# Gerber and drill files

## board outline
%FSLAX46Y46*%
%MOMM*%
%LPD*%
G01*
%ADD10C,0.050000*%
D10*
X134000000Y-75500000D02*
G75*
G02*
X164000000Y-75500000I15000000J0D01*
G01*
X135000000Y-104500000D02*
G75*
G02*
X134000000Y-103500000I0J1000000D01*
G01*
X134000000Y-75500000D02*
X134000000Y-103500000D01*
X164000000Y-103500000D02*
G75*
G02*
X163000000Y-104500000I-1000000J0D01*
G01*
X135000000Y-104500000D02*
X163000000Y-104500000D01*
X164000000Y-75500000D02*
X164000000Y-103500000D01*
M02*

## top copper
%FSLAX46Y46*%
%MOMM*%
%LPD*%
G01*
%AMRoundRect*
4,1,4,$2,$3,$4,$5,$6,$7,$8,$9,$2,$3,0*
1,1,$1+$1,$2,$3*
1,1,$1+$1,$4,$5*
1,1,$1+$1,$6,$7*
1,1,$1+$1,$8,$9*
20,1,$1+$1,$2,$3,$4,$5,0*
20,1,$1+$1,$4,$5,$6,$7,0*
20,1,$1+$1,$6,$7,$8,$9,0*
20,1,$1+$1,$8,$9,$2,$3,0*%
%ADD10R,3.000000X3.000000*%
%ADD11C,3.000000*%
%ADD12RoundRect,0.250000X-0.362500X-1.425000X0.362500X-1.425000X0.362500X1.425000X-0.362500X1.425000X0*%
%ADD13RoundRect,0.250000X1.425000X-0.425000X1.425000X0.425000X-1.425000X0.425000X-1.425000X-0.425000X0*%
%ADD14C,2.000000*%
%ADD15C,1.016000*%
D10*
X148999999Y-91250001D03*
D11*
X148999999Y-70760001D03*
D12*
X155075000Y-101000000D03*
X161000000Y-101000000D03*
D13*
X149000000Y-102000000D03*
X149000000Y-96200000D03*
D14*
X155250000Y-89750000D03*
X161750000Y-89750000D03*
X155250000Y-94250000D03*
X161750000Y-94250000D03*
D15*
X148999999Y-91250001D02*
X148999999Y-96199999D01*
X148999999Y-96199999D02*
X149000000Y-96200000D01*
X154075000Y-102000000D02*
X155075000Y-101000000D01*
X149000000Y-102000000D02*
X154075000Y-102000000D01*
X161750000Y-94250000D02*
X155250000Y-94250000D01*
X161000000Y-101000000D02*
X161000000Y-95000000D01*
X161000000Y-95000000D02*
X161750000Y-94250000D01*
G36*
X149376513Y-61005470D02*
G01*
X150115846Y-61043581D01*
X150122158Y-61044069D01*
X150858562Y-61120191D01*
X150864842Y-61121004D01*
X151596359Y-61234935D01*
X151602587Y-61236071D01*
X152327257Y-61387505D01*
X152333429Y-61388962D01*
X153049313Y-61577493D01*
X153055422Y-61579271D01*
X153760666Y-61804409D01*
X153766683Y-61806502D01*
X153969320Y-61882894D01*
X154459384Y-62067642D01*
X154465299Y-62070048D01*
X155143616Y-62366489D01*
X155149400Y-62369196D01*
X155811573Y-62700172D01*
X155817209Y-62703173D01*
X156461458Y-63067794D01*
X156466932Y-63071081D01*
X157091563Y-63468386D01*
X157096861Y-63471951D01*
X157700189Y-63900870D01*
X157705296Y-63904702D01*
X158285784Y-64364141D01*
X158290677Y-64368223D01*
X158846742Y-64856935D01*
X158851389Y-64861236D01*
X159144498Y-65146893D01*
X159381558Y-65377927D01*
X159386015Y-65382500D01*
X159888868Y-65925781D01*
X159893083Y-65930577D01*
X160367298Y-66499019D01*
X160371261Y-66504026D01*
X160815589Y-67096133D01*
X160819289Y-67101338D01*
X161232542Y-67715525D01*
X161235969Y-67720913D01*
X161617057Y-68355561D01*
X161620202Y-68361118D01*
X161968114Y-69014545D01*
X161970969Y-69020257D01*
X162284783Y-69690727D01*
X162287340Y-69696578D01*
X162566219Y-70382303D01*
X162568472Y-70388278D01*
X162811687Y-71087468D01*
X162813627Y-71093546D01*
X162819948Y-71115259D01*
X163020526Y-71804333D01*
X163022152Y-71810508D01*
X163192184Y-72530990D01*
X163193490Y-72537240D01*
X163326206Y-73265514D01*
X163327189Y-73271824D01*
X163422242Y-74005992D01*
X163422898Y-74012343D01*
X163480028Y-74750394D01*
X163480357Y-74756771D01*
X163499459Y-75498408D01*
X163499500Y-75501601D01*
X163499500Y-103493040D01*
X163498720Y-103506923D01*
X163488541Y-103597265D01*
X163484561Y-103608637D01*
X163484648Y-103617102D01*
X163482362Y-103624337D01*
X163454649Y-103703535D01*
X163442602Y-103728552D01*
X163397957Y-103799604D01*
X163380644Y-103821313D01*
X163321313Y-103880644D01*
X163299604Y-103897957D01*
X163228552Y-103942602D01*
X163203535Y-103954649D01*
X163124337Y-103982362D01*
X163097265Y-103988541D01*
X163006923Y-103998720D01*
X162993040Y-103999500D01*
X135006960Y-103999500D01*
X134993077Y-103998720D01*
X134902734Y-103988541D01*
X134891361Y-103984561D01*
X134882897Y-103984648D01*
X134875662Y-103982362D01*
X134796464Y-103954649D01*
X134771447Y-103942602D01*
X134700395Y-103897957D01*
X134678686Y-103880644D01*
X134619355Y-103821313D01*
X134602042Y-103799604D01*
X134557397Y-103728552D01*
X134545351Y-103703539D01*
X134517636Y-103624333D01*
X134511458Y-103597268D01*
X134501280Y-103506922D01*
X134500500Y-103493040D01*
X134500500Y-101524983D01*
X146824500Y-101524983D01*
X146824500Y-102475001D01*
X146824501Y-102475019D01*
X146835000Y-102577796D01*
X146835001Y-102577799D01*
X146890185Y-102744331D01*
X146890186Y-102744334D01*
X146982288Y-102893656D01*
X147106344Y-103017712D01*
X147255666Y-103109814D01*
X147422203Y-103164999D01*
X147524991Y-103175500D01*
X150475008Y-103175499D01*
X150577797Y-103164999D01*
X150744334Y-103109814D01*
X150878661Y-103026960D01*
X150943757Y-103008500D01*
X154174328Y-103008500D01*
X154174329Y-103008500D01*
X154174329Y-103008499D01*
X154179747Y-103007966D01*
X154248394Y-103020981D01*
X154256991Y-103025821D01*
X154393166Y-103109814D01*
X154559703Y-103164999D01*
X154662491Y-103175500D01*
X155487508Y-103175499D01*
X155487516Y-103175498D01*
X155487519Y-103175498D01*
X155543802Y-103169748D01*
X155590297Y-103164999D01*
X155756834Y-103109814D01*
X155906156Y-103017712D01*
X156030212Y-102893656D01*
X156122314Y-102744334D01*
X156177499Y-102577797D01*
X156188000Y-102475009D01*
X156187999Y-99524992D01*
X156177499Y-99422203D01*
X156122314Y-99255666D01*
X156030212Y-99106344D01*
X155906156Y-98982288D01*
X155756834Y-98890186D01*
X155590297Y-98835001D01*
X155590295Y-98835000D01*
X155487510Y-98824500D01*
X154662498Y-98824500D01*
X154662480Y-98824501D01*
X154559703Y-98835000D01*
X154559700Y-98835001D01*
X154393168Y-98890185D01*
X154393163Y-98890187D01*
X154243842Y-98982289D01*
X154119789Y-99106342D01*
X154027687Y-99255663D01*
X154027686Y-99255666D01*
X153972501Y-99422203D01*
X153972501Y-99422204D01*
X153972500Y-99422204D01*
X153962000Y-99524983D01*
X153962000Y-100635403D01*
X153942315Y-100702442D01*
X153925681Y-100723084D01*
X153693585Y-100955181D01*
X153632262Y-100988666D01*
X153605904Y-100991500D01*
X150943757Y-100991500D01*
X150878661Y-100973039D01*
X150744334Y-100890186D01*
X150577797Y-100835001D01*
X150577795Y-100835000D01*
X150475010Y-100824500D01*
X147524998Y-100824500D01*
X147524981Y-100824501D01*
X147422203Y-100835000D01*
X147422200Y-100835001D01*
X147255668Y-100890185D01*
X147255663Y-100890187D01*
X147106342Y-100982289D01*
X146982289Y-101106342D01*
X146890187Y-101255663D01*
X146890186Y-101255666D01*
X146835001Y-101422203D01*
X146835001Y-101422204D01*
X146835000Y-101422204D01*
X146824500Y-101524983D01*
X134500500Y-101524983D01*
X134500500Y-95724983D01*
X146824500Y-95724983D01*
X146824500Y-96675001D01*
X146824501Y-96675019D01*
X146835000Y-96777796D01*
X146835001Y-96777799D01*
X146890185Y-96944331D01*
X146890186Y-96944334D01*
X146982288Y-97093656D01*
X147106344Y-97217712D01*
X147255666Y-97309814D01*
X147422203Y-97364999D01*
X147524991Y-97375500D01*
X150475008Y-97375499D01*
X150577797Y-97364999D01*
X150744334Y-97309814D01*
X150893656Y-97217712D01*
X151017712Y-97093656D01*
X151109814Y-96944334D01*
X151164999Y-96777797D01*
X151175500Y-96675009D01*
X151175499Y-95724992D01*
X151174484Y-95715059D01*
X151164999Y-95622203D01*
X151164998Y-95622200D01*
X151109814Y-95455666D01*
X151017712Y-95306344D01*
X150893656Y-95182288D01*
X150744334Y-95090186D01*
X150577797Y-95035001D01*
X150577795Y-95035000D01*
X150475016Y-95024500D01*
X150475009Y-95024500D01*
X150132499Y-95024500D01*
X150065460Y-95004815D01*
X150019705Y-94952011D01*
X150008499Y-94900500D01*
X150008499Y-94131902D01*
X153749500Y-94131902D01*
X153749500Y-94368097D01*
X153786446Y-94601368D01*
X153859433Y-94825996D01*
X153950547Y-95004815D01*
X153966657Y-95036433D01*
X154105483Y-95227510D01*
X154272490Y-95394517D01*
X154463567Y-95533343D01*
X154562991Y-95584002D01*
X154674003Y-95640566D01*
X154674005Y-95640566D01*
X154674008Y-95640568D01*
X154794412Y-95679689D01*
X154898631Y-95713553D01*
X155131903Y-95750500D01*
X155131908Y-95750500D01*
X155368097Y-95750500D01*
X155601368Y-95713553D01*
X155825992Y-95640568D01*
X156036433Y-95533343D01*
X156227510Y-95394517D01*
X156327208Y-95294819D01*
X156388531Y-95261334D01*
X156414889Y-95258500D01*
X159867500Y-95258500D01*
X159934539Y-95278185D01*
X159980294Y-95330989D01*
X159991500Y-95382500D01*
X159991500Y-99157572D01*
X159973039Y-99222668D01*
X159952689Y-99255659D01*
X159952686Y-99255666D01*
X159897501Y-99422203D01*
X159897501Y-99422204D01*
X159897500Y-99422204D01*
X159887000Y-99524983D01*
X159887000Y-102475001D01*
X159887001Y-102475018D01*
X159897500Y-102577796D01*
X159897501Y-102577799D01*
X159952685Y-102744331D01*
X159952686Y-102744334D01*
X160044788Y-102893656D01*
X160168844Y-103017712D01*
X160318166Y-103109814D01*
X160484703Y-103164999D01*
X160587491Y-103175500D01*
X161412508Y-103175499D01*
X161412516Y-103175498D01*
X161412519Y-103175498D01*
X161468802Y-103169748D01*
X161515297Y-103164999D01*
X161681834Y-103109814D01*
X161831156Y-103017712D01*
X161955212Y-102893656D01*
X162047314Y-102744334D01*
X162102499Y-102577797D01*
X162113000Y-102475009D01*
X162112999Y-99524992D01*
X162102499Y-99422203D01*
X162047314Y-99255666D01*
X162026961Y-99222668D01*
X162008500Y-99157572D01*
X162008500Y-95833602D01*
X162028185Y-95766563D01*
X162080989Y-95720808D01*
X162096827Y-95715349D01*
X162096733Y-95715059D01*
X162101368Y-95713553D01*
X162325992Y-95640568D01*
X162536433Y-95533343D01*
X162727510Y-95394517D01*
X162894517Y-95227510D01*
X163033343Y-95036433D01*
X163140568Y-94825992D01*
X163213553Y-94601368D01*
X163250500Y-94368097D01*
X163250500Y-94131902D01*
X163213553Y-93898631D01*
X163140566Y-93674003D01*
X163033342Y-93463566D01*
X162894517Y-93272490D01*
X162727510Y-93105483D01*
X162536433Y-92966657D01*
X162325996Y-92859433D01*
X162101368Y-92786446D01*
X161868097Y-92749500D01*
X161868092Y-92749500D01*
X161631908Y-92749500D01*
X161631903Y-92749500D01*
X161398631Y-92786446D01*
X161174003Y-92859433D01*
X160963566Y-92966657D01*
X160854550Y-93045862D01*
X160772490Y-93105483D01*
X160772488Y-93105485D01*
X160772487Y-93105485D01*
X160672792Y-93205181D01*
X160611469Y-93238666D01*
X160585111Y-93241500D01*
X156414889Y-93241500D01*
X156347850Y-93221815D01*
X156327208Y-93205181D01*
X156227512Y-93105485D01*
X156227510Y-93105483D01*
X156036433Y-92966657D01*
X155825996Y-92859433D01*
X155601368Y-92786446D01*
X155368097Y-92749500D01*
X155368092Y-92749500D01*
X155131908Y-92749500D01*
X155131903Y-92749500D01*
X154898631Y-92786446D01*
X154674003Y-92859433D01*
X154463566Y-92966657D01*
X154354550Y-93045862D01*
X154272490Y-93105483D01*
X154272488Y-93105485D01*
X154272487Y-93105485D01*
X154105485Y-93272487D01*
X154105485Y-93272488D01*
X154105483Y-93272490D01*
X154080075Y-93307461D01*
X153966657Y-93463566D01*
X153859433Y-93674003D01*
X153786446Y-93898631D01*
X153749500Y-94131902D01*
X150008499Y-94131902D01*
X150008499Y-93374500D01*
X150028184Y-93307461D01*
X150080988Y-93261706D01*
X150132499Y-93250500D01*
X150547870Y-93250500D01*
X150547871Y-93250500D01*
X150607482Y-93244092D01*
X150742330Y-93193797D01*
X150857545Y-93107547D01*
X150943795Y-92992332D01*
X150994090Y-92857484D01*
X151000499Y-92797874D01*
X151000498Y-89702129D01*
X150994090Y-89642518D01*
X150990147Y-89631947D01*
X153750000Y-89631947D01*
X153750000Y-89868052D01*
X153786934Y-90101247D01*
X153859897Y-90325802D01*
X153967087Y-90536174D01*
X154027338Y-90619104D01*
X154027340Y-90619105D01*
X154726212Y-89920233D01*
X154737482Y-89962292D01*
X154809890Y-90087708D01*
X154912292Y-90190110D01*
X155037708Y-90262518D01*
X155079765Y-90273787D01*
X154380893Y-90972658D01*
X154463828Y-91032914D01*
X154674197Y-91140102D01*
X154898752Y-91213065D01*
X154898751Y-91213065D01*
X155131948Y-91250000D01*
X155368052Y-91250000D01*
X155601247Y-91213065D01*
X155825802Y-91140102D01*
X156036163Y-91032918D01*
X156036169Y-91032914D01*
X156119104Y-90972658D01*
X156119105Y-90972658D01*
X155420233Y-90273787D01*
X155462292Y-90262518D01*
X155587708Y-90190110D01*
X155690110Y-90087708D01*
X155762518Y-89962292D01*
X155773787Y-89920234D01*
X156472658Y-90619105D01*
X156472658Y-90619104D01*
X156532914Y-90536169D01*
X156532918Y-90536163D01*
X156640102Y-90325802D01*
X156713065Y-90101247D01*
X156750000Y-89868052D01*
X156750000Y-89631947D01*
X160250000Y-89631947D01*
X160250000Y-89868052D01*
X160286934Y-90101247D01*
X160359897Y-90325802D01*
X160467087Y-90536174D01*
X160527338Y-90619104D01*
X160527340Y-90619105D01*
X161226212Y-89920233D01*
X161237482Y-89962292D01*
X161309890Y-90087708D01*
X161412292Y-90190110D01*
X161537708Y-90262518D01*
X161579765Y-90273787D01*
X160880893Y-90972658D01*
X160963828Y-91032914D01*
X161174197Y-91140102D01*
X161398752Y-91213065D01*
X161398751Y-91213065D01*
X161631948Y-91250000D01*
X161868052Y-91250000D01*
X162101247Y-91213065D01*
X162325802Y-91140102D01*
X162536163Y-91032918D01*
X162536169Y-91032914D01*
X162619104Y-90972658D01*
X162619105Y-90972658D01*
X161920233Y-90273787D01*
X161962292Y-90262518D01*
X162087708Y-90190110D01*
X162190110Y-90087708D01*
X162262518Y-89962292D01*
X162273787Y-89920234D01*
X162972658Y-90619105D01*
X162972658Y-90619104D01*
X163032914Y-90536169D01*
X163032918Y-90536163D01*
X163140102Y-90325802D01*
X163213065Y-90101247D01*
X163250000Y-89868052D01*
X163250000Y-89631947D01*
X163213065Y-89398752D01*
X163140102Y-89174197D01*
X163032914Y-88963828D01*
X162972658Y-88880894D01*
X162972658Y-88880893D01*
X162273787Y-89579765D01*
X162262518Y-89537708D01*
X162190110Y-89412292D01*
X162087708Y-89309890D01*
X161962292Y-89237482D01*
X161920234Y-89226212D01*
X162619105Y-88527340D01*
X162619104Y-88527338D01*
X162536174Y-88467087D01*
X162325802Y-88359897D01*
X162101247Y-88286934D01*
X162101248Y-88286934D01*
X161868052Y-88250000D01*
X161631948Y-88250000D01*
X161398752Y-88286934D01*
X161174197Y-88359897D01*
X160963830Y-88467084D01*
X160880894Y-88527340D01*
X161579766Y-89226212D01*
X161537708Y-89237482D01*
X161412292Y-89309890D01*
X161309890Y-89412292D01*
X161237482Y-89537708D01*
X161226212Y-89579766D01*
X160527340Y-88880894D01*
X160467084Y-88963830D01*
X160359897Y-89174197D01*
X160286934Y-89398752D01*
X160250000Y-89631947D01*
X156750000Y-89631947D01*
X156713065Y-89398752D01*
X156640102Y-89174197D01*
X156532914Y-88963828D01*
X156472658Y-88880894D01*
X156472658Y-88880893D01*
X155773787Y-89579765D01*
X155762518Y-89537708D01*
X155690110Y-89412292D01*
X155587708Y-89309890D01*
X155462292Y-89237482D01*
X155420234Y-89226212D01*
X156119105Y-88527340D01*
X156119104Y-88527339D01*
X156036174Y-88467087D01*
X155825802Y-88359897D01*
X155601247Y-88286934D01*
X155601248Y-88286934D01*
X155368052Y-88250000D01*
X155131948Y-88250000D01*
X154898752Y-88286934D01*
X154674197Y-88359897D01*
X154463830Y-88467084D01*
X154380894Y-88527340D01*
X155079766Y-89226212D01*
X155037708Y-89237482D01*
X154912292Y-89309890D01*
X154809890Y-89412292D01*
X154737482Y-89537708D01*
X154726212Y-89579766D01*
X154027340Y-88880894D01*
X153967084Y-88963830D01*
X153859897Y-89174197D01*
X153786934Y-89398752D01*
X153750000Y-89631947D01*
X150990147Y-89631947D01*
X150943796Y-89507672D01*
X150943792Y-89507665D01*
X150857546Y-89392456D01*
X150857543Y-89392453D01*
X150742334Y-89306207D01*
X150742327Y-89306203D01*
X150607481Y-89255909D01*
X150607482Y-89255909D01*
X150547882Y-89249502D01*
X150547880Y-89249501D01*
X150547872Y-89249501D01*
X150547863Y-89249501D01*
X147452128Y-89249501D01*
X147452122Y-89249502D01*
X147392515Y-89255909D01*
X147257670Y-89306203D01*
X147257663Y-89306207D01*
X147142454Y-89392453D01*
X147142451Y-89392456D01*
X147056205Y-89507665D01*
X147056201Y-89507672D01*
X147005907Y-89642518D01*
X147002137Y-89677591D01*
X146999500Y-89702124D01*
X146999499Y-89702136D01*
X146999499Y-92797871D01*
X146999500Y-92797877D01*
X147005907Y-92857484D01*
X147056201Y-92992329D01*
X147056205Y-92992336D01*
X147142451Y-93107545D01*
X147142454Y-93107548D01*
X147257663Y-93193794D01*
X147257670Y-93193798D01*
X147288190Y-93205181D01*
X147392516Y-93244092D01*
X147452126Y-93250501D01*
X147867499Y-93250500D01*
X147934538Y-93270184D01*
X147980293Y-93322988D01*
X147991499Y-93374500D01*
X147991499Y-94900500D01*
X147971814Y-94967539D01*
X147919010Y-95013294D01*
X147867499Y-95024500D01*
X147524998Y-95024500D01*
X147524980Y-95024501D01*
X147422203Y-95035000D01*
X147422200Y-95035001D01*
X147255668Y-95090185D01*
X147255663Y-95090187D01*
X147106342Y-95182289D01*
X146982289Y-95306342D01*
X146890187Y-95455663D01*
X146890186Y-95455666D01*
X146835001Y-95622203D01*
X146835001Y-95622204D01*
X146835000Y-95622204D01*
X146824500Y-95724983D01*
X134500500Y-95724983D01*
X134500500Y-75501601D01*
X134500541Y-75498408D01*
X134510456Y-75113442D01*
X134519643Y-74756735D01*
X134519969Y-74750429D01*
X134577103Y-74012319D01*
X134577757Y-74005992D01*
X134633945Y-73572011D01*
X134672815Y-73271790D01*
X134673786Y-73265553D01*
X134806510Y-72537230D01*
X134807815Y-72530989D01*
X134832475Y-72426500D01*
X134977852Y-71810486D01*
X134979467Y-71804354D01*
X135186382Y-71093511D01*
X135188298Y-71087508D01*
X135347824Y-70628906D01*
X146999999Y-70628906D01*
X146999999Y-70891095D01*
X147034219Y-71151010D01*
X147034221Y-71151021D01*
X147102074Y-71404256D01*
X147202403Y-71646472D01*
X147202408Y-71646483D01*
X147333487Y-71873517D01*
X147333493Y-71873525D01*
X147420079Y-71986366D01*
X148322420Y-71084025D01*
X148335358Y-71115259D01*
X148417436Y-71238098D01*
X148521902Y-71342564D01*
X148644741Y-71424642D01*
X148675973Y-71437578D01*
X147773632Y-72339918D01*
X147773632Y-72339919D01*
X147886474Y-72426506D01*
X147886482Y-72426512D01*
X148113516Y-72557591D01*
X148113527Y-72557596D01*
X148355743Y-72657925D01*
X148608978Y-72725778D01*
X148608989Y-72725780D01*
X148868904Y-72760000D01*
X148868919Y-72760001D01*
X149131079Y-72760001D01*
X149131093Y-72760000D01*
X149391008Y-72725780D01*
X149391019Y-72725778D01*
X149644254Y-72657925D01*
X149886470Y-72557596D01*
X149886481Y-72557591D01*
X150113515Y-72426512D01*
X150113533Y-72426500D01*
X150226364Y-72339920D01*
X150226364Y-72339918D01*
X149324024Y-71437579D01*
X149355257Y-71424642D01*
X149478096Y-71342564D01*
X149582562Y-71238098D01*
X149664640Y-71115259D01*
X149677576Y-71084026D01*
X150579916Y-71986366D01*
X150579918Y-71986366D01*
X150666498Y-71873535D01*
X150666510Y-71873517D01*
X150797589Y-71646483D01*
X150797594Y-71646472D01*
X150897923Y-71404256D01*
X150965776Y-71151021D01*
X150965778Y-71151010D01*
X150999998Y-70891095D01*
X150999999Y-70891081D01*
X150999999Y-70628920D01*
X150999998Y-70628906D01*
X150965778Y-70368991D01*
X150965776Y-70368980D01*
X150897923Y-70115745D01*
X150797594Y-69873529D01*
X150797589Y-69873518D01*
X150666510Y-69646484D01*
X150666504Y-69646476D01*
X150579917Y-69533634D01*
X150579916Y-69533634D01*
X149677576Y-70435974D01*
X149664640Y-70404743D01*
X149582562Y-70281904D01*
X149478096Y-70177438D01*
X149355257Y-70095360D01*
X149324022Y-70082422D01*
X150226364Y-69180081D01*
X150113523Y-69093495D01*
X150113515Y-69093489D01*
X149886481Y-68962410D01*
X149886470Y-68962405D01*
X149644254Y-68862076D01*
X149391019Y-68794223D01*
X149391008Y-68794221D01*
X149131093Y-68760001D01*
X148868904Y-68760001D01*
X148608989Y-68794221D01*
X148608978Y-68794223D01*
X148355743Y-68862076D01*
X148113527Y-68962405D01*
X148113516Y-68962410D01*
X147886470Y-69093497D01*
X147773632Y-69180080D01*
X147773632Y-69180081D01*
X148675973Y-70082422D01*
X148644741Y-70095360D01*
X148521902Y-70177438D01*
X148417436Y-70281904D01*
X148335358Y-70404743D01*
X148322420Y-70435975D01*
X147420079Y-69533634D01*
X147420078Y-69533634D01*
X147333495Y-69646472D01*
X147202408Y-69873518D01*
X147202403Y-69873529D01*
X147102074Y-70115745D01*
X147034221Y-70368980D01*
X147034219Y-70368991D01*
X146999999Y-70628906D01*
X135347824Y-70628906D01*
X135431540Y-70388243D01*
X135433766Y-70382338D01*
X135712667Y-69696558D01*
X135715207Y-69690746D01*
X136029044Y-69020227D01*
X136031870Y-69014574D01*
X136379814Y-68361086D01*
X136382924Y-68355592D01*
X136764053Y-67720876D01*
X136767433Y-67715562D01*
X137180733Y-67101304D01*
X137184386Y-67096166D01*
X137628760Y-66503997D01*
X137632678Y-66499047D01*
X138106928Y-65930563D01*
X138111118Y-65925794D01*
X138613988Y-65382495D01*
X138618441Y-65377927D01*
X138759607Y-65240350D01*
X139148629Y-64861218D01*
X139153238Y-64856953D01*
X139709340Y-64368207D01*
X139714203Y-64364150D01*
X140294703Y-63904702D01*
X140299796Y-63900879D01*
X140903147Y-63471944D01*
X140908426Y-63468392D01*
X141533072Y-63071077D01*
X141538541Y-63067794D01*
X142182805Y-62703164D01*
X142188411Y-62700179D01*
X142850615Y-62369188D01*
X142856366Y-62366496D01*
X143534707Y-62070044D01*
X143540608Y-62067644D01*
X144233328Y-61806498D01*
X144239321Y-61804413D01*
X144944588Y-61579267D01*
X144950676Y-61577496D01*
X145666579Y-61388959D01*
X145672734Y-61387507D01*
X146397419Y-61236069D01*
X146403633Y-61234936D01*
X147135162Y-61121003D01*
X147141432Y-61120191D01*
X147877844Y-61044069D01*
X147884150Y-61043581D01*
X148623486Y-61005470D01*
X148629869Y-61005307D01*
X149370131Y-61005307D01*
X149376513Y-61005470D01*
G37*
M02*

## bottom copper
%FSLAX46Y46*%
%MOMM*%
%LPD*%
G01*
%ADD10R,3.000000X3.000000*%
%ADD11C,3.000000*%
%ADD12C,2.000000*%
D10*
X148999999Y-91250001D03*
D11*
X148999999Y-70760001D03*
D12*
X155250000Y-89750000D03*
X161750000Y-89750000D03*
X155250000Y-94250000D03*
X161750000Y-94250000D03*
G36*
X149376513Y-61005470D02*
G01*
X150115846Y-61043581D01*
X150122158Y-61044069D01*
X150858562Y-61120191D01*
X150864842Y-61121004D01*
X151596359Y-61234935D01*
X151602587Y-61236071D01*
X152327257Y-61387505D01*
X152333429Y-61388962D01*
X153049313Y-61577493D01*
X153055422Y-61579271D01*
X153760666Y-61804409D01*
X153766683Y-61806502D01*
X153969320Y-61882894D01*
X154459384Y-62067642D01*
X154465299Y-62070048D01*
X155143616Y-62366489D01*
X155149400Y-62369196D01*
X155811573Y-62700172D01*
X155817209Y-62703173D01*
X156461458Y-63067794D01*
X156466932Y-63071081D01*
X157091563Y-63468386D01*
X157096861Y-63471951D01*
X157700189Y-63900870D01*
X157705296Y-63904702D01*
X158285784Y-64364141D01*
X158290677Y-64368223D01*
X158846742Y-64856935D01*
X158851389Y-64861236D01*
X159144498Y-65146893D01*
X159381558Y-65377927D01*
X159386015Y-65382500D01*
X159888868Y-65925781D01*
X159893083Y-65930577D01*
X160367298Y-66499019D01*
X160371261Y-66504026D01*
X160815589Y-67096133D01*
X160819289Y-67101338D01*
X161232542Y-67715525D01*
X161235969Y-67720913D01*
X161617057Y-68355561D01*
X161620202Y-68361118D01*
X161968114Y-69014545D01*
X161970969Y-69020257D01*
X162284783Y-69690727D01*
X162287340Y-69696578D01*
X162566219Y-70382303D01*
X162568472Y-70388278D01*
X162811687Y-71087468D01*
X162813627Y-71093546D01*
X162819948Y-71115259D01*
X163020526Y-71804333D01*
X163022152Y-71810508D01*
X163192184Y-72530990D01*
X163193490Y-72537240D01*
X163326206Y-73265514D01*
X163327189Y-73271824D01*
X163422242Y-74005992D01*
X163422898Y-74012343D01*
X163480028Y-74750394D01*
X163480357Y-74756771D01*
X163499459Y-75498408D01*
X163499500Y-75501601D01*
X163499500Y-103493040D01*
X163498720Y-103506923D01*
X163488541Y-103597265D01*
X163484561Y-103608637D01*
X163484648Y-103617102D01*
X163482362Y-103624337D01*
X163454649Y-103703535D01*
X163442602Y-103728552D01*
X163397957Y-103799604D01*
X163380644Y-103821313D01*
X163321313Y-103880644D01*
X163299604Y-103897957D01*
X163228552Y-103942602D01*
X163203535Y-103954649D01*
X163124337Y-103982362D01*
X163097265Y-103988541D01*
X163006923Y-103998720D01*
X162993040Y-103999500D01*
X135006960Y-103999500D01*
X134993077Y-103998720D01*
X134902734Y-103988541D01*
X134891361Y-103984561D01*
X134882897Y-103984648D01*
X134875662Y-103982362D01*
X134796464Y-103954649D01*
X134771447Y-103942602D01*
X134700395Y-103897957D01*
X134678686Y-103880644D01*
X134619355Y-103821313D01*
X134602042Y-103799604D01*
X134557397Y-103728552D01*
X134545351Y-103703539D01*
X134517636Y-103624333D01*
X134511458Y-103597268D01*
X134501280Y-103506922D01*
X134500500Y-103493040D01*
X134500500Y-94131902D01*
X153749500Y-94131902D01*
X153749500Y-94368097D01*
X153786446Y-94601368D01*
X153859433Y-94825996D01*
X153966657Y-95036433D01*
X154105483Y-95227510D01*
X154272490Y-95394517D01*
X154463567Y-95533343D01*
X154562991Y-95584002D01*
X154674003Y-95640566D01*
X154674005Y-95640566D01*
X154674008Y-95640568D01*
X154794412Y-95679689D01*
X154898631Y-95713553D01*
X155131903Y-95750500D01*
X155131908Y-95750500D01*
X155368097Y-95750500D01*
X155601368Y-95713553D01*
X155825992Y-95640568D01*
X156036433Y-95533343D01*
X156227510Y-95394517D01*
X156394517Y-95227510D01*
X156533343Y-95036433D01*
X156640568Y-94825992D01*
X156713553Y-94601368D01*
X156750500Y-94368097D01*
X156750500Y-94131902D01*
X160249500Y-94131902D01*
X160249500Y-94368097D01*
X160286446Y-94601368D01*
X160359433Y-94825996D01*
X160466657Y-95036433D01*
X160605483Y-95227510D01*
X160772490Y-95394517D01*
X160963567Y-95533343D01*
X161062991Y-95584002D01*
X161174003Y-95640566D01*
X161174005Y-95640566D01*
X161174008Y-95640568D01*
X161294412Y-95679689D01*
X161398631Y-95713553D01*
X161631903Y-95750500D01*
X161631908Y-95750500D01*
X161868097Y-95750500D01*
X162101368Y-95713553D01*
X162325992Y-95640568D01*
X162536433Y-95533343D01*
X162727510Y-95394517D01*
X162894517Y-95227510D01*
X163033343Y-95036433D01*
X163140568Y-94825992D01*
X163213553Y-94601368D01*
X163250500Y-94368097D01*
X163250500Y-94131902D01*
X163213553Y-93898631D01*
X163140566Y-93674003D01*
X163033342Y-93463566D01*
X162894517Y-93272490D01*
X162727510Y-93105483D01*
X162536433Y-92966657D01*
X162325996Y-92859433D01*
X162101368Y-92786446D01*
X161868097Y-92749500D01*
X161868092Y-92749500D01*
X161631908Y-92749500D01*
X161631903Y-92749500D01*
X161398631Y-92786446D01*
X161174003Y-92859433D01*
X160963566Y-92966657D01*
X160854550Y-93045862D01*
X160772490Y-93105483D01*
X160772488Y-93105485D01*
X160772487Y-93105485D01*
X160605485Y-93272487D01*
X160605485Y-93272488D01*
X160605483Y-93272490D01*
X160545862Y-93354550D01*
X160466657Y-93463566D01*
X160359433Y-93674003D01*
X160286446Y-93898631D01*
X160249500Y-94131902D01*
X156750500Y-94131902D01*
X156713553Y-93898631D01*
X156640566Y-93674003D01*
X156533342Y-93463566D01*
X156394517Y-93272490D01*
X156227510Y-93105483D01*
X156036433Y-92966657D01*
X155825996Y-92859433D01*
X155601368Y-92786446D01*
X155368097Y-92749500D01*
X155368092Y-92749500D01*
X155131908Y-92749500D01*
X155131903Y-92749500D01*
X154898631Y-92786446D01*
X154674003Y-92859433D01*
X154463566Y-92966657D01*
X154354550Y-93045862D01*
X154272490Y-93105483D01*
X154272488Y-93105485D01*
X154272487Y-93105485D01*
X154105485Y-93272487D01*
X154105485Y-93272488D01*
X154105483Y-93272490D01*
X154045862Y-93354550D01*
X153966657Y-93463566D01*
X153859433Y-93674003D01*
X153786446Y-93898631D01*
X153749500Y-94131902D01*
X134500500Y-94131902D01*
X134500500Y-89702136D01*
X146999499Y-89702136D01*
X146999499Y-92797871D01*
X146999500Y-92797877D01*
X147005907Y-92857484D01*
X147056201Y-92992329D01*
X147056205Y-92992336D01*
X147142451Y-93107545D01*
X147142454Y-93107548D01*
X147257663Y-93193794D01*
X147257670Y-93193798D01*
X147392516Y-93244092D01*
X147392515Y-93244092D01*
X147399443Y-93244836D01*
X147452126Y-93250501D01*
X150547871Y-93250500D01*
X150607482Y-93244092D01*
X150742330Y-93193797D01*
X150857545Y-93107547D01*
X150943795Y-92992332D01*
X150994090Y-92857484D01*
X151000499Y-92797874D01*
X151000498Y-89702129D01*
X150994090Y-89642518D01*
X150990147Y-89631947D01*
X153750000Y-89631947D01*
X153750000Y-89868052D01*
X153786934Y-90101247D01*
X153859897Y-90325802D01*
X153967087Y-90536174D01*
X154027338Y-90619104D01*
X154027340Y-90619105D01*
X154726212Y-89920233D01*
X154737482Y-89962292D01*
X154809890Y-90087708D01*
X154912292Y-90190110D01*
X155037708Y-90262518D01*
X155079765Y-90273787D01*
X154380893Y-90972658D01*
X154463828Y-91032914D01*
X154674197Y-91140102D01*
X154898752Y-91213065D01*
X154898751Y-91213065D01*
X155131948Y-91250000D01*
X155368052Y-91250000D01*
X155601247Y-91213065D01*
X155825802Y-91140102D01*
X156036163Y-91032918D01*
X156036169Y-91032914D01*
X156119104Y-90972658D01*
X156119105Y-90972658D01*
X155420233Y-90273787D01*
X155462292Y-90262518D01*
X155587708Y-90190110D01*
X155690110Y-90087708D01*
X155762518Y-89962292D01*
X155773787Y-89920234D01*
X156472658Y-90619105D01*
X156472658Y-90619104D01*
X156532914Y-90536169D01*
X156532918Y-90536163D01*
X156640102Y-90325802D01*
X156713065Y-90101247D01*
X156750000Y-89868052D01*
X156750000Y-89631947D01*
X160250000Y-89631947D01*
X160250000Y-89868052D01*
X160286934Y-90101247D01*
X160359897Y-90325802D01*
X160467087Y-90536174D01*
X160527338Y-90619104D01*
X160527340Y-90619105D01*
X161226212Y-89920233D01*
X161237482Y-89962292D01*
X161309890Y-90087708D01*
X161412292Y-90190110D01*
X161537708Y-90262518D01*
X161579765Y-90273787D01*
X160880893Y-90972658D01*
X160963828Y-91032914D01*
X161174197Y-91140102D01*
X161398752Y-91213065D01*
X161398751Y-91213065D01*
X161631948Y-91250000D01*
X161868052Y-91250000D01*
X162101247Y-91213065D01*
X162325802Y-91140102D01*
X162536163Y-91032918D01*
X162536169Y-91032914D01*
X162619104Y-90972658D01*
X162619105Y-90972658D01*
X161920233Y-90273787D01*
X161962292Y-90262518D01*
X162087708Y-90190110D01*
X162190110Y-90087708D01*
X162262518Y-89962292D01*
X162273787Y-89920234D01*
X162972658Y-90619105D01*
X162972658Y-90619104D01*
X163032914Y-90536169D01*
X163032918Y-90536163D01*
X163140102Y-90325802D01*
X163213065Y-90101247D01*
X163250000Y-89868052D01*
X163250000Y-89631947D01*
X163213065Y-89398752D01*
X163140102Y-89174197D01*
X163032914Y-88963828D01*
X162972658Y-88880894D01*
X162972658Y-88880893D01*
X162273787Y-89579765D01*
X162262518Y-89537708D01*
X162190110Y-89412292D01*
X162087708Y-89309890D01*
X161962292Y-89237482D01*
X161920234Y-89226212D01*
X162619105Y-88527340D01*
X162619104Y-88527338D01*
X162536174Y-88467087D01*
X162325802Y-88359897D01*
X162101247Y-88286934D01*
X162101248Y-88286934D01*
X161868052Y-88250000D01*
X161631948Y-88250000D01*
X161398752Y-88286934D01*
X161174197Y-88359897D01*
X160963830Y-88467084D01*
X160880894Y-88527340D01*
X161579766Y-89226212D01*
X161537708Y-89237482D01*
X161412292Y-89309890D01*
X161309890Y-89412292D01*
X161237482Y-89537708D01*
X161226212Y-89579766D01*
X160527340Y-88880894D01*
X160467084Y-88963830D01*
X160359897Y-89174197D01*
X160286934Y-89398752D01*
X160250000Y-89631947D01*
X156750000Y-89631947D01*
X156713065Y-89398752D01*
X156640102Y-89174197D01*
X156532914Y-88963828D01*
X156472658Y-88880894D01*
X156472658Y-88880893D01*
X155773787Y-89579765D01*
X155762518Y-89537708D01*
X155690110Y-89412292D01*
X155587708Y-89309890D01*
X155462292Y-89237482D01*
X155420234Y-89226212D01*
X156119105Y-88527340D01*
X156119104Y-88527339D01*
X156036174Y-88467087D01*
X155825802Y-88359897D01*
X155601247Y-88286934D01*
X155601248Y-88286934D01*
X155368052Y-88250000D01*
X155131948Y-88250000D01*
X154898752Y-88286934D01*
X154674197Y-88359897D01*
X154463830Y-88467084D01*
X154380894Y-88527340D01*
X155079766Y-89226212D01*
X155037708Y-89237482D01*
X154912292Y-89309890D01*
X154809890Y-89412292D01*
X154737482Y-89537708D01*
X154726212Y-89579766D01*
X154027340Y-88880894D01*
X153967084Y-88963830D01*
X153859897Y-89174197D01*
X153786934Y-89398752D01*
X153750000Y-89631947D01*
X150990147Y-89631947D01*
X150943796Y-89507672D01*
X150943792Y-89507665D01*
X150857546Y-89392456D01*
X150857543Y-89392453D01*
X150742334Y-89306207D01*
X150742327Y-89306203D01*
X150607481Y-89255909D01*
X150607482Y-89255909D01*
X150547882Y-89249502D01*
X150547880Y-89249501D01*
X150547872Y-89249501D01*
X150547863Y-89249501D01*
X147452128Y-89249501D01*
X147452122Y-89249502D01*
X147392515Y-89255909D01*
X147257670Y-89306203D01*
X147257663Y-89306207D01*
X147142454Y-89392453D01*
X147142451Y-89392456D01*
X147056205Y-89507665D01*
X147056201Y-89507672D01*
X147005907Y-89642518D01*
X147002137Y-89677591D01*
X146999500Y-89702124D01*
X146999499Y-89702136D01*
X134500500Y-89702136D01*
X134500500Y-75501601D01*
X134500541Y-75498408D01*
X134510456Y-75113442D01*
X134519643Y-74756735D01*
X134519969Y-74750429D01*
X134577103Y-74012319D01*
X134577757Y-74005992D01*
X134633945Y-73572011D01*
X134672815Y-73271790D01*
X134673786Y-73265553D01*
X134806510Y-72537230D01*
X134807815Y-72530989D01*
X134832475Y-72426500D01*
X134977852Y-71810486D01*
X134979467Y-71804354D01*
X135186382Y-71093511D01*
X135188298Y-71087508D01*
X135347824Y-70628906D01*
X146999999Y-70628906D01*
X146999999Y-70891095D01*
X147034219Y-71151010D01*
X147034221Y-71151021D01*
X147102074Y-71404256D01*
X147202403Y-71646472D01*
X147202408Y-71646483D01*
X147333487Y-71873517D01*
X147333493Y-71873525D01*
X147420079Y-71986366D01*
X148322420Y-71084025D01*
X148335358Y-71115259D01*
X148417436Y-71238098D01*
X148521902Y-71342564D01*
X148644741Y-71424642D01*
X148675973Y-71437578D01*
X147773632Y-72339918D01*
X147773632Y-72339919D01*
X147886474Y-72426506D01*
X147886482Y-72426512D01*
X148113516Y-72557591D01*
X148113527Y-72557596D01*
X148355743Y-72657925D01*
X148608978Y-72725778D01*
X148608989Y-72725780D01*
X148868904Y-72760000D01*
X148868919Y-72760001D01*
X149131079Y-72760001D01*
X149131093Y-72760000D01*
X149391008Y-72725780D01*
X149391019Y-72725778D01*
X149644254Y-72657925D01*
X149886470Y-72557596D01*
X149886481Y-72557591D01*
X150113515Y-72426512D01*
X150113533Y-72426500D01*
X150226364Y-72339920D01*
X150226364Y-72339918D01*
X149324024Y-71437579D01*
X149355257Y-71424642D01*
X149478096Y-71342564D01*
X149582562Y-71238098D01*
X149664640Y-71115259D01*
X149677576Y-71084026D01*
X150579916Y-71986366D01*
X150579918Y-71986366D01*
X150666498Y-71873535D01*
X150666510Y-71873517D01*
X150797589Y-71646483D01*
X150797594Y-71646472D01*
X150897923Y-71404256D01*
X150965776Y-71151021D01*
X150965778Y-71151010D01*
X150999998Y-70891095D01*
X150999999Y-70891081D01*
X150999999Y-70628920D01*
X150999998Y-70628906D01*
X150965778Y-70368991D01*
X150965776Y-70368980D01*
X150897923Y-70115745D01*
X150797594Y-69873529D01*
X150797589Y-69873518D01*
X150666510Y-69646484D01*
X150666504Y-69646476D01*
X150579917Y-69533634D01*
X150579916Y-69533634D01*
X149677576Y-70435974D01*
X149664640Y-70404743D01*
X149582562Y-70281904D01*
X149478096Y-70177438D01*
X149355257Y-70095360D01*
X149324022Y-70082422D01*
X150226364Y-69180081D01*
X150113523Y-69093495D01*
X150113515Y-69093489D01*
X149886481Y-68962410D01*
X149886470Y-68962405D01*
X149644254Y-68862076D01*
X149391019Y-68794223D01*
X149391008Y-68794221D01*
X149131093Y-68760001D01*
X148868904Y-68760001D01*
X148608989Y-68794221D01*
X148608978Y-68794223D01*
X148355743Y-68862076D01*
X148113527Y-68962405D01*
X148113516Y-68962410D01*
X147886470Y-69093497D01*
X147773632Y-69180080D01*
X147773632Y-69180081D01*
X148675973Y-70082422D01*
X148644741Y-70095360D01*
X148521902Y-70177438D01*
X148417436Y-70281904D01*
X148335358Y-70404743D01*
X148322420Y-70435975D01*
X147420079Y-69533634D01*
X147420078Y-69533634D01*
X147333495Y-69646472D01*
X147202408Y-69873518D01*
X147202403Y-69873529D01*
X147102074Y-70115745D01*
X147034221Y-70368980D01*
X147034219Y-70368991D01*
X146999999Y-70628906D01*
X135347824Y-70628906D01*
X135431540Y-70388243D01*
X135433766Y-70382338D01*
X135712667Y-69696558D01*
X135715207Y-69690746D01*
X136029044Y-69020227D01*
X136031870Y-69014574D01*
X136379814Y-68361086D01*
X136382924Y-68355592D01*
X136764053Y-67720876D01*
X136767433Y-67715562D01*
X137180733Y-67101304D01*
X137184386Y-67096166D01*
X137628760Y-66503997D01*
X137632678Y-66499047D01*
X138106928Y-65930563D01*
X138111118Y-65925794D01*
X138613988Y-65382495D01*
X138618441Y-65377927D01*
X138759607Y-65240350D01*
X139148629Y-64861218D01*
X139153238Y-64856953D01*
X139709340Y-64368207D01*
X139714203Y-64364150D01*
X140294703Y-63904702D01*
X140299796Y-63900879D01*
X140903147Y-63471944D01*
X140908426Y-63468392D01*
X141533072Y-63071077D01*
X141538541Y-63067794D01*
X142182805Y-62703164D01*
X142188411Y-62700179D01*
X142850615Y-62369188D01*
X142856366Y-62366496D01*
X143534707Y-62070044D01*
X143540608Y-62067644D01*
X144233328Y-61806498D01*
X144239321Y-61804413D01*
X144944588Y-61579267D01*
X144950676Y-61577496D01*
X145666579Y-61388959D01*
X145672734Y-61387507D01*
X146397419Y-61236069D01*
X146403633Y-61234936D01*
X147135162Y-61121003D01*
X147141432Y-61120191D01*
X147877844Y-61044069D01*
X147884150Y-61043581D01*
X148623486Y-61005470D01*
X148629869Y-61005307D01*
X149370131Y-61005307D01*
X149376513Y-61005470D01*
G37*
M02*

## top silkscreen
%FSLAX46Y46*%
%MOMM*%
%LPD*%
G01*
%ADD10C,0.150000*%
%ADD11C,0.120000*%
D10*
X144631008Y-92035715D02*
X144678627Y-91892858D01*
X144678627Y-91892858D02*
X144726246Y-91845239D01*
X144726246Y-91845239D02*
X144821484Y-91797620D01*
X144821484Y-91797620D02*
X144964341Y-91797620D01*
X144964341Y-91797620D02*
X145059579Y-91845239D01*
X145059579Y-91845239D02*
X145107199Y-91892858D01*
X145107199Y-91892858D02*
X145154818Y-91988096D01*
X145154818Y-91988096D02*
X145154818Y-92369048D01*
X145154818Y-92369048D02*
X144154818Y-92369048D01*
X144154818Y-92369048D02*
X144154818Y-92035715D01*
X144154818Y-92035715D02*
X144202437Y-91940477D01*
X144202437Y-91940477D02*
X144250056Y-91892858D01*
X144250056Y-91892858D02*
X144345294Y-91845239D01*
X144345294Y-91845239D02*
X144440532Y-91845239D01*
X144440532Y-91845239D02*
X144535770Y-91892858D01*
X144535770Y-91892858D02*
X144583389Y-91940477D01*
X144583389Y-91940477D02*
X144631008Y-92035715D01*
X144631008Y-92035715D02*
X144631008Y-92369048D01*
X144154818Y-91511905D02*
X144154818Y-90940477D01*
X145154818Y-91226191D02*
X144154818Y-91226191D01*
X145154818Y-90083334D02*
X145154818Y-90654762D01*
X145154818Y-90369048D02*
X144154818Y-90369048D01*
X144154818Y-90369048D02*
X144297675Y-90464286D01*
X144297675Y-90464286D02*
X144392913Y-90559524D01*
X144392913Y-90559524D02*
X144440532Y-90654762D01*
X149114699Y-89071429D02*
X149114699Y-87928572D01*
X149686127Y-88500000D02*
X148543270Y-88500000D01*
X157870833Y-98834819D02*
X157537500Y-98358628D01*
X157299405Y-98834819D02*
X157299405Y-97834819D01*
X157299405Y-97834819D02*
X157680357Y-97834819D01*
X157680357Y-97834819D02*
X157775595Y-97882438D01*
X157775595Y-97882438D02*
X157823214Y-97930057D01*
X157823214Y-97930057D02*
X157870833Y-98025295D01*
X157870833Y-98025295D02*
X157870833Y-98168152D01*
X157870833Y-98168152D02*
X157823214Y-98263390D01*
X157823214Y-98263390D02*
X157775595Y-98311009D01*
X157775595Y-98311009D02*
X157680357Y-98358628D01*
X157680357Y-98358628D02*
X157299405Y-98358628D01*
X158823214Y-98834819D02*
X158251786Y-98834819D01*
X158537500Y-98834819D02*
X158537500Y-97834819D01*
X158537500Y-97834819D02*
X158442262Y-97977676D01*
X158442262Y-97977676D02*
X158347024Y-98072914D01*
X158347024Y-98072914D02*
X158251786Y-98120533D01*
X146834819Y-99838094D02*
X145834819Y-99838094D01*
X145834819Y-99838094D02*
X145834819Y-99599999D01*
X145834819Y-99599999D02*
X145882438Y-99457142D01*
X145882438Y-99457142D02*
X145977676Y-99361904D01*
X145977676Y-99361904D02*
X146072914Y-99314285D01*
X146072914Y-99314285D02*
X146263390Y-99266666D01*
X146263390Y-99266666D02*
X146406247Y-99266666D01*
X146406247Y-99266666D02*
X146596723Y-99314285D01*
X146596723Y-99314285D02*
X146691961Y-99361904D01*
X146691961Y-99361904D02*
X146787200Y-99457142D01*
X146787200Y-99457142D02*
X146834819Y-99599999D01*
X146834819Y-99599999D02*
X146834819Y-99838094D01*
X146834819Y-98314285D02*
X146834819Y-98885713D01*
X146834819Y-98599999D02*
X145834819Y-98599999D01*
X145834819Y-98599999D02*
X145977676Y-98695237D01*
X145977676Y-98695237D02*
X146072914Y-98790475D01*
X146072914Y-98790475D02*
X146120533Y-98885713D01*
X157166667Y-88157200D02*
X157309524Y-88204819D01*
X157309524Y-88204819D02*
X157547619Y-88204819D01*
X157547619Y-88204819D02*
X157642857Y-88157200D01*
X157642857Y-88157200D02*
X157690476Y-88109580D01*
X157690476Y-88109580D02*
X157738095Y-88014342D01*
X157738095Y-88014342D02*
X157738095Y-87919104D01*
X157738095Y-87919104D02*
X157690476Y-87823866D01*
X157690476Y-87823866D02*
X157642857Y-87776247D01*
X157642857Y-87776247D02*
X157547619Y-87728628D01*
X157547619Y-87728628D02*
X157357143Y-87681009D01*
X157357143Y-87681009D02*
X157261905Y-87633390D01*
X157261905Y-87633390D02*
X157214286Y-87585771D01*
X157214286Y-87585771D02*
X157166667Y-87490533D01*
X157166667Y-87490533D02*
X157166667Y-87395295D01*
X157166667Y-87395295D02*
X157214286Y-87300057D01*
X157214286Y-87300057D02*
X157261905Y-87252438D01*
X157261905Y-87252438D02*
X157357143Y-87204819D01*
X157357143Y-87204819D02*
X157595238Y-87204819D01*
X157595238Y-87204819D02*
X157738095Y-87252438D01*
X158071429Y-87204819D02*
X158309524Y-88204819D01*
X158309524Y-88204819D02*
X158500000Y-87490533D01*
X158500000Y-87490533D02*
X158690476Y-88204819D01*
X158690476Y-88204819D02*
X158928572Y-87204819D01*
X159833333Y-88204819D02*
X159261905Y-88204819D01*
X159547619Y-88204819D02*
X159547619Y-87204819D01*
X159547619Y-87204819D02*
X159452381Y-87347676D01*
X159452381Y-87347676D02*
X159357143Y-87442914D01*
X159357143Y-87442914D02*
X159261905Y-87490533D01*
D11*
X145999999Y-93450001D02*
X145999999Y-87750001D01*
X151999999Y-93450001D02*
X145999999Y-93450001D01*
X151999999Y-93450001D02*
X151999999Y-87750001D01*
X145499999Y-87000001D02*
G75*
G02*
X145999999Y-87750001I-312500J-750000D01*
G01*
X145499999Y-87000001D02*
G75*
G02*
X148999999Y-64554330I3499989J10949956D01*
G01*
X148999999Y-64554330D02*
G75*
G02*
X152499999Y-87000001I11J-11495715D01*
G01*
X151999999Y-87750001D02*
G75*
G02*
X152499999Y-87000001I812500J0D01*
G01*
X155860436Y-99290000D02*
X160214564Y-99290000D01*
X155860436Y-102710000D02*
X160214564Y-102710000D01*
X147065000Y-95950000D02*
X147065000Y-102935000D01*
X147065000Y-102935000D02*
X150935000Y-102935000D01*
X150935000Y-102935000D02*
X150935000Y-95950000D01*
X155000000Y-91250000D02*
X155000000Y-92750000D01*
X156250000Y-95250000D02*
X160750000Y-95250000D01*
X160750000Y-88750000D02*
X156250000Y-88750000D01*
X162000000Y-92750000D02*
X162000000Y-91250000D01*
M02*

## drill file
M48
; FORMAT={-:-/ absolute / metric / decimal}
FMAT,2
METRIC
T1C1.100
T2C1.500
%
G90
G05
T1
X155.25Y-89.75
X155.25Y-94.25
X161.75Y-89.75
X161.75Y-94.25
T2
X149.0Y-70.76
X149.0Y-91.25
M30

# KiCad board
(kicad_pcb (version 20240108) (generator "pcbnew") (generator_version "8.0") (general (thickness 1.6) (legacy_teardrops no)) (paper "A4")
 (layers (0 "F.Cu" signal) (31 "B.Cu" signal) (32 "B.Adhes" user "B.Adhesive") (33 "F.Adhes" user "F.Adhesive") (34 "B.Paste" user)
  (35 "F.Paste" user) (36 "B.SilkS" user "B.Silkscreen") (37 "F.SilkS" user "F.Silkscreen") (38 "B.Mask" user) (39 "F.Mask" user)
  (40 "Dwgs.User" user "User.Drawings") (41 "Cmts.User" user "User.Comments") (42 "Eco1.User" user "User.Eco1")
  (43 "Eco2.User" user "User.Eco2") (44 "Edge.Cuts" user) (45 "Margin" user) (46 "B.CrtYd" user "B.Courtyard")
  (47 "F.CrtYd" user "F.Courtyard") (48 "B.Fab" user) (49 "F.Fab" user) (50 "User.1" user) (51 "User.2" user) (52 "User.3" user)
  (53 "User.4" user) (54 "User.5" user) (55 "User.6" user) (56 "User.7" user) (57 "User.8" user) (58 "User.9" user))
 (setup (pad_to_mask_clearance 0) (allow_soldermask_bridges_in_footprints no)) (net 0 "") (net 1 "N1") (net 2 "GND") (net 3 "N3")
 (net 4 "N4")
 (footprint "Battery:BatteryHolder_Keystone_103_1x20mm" (layer "F.Cu") (at 148.999999 91.250001 90)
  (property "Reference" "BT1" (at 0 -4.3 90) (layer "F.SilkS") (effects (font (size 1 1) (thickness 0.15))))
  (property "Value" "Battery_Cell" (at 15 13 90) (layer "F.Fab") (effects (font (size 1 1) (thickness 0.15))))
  (fp_line (start -2.2 -3) (end 3.5 -3) (stroke (width 0.12) (type solid)) (layer "F.SilkS"))
  (fp_line (start -2.2 3) (end -2.2 -3) (stroke (width 0.12) (type solid)) (layer "F.SilkS"))
  (fp_line (start -2.2 3) (end 3.5 3) (stroke (width 0.12) (type solid)) (layer "F.SilkS"))
  (fp_arc (start 4.25 -3.5) (mid 3.950694 -3.136459) (end 3.5 -3) (stroke (width 0.12) (type solid)) (layer "F.SilkS"))
  (fp_arc (start 4.25 -3.5) (mid 16.971103 -11.358466) (end 26.695671 0) (stroke (width 0.12) (type solid)) (layer "F.SilkS"))
  (fp_arc (start 26.695671 0) (mid 16.971103 11.358466) (end 4.25 3.5) (stroke (width 0.12) (type solid)) (layer "F.SilkS"))
  (fp_arc (start 3.5 3) (mid 3.950694 3.136459) (end 4.25 3.5) (stroke (width 0.12) (type solid)) (layer "F.SilkS"))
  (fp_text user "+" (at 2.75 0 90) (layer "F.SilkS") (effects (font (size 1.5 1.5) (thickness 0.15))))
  (pad "1" thru_hole rect (at 0 0 90) (size 3 3) (drill 1.5) (layers "*.Cu" "*.Mask") (remove_unused_layers no) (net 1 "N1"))
  (pad "2" thru_hole circle (at 20.49 0 90) (size 3 3) (drill 1.5) (layers "*.Cu" "*.Mask") (remove_unused_layers no) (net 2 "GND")))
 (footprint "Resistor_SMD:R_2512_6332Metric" (layer "F.Cu") (at 158.0375 101)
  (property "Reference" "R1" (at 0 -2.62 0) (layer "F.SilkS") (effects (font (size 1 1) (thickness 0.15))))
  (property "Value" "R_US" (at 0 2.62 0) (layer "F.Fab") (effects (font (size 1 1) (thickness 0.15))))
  (fp_line (start -2.177064 -1.71) (end 2.177064 -1.71) (stroke (width 0.12) (type solid)) (layer "F.SilkS"))
  (fp_line (start -2.177064 1.71) (end 2.177064 1.71) (stroke (width 0.12) (type solid)) (layer "F.SilkS"))
  (pad "1" smd roundrect (at -2.9625 0) (size 1.225 3.35) (layers "F.Cu" "F.Paste" "F.Mask") (roundrect_rratio 0.204082) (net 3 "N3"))
  (pad "2" smd roundrect (at 2.9625 0) (size 1.225 3.35) (layers "F.Cu" "F.Paste" "F.Mask") (roundrect_rratio 0.204082) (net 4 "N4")))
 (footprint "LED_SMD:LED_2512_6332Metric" (layer "F.Cu") (at 149 99.1 90)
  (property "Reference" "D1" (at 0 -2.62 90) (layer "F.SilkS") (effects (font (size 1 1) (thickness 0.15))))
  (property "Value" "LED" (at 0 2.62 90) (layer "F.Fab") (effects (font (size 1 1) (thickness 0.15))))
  (fp_line (start 3.15 -1.935) (end -3.835 -1.935) (stroke (width 0.12) (type solid)) (layer "F.SilkS"))
  (fp_line (start -3.835 -1.935) (end -3.835 1.935) (stroke (width 0.12) (type solid)) (layer "F.SilkS"))
  (fp_line (start -3.835 1.935) (end 3.15 1.935) (stroke (width 0.12) (type solid)) (layer "F.SilkS"))
  (pad "1" smd roundrect (at -2.9 0 90) (size 1.35 3.35) (layers "F.Cu" "F.Paste" "F.Mask") (roundrect_rratio 0.185185) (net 3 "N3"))
  (pad "2" smd roundrect (at 2.9 0 90) (size 1.35 3.35) (layers "F.Cu" "F.Paste" "F.Mask") (roundrect_rratio 0.185185) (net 1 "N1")))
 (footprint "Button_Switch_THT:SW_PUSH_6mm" (layer "F.Cu") (at 155.25 89.75)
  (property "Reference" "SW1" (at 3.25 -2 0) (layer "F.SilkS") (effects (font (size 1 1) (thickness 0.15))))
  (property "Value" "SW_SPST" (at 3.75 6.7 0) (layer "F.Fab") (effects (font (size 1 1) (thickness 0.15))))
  (fp_line (start -0.25 1.5) (end -0.25 3) (stroke (width 0.12) (type solid)) (layer "F.SilkS"))
  (fp_line (start 1 5.5) (end 5.5 5.5) (stroke (width 0.12) (type solid)) (layer "F.SilkS"))
  (fp_line (start 5.5 -1) (end 1 -1) (stroke (width 0.12) (type solid)) (layer "F.SilkS"))
  (fp_line (start 6.75 3) (end 6.75 1.5) (stroke (width 0.12) (type solid)) (layer "F.SilkS"))
  (pad "1" thru_hole circle (at 0 0 90) (size 2 2) (drill 1.1) (layers "*.Cu" "*.Mask") (remove_unused_layers no) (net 2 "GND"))
  (pad "1" thru_hole circle (at 6.5 0 90) (size 2 2) (drill 1.1) (layers "*.Cu" "*.Mask") (remove_unused_layers no) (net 2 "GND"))
  (pad "2" thru_hole circle (at 0 4.5 90) (size 2 2) (drill 1.1) (layers "*.Cu" "*.Mask") (remove_unused_layers no) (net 4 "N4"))
  (pad "2" thru_hole circle (at 6.5 4.5 90) (size 2 2) (drill 1.1) (layers "*.Cu" "*.Mask") (remove_unused_layers no) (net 4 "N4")))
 (gr_arc (start 134 75.5) (mid 149 60.5) (end 164 75.5) (stroke (width 0.05) (type default)) (layer "Edge.Cuts"))
 (gr_arc (start 135 104.5) (mid 134.292893 104.207107) (end 134 103.5) (stroke (width 0.05) (type default)) (layer "Edge.Cuts"))
 (gr_line (start 134 75.5) (end 134 103.5) (stroke (width 0.05) (type default)) (layer "Edge.Cuts"))
 (gr_arc (start 164 103.5) (mid 163.707107 104.207107) (end 163 104.5) (stroke (width 0.05) (type default)) (layer "Edge.Cuts"))
 (gr_line (start 135 104.5) (end 163 104.5) (stroke (width 0.05) (type default)) (layer "Edge.Cuts"))
 (gr_line (start 164 75.5) (end 164 103.5) (stroke (width 0.05) (type default)) (layer "Edge.Cuts"))
 (segment (start 148.999999 91.250001) (end 148.999999 96.199999) (width 1.016) (layer "F.Cu") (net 1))
 (segment (start 148.999999 96.199999) (end 149 96.2) (width 1.016) (layer "F.Cu") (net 1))
 (segment (start 154.075 102) (end 155.075 101) (width 1.016) (layer "F.Cu") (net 3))
 (segment (start 149 102) (end 154.075 102) (width 1.016) (layer "F.Cu") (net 3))
 (segment (start 161.75 94.25) (end 155.25 94.25) (width 1.016) (layer "F.Cu") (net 4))
 (segment (start 161 101) (end 161 95) (width 1.016) (layer "F.Cu") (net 4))
 (segment (start 161 95) (end 161.75 94.25) (width 1.016) (layer "F.Cu") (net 4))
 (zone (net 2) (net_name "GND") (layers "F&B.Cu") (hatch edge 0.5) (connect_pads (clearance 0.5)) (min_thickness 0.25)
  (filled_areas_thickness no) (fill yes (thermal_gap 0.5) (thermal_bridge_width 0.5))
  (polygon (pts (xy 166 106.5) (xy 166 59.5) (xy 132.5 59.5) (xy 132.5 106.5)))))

